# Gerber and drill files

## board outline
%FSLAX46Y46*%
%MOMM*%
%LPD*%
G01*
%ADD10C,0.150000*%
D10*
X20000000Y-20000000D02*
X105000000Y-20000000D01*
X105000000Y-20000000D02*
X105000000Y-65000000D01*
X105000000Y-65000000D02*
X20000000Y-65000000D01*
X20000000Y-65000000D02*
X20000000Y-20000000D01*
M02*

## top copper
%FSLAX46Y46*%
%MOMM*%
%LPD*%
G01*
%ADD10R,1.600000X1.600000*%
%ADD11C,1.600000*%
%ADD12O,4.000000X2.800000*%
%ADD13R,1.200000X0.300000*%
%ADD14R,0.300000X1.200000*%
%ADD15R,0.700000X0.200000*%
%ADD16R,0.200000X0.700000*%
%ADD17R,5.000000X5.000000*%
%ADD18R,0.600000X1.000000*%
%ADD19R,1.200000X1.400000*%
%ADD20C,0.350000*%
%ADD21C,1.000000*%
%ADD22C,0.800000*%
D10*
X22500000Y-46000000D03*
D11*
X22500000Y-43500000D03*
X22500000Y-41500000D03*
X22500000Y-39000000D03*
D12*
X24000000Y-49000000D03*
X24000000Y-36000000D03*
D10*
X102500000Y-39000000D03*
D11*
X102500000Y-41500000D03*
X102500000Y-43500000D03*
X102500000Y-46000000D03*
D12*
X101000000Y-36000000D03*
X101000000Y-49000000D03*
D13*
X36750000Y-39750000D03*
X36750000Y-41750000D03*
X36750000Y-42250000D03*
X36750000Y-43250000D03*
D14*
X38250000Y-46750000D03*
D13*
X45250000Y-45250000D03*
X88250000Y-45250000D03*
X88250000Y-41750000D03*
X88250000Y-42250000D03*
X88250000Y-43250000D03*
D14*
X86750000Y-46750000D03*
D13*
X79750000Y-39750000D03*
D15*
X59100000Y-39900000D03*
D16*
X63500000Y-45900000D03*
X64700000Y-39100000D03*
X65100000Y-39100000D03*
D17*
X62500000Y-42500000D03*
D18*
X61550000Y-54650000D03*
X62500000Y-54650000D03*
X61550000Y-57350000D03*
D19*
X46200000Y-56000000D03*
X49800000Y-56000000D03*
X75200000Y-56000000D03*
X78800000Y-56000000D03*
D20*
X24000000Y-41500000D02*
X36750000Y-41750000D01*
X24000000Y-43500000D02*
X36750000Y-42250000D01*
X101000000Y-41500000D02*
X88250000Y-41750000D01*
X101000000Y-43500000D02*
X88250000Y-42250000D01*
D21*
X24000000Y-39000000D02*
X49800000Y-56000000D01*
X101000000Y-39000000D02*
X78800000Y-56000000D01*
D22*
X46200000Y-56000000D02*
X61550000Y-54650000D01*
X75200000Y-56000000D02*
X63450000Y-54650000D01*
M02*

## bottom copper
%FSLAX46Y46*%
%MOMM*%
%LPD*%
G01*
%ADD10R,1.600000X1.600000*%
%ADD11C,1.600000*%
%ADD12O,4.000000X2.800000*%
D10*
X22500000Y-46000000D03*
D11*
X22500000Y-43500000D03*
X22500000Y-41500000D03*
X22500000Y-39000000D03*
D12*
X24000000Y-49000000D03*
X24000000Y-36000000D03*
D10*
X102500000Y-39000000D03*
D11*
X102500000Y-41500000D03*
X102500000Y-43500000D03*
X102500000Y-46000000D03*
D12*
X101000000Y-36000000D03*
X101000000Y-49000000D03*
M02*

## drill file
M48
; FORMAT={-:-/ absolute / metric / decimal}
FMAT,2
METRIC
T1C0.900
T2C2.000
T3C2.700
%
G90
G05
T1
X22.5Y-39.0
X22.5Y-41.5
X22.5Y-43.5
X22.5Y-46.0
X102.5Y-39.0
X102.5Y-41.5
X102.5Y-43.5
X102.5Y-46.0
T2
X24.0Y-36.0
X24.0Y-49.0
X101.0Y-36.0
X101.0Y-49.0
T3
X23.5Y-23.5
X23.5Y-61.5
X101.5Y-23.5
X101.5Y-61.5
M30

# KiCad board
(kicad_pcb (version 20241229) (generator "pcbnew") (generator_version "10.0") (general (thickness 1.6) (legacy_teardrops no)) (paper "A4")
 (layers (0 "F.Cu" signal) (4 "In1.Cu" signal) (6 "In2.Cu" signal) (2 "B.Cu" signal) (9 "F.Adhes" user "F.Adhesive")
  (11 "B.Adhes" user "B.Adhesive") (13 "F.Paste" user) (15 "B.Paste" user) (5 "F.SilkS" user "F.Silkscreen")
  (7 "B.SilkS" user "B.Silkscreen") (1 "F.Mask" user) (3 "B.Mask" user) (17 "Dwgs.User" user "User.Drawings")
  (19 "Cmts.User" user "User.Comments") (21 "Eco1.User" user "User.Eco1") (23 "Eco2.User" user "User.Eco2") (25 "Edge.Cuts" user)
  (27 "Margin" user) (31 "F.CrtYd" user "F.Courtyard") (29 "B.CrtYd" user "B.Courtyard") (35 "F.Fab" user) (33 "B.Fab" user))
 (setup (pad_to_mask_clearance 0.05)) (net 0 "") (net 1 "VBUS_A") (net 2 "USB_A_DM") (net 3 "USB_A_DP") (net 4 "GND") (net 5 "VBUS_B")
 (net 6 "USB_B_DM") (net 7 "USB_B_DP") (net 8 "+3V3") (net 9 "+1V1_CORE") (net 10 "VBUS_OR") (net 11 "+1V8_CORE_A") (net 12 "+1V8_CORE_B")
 (gr_line (start 20.0 20.0) (end 105.0 20.0) (layer "Edge.Cuts") (width 0.15))
 (gr_line (start 105.0 20.0) (end 105.0 65.0) (layer "Edge.Cuts") (width 0.15))
 (gr_line (start 105.0 65.0) (end 20.0 65.0) (layer "Edge.Cuts") (width 0.15))
 (gr_line (start 20.0 65.0) (end 20.0 20.0) (layer "Edge.Cuts") (width 0.15))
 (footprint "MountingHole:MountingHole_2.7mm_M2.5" (layer "F.Cu") (at 23.5 23.5)
  (pad "1" np_thru_hole circle (at 0 0) (size 2.7 2.7) (drill 2.7) (layers "*.Mask")))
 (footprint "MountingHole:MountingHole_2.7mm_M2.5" (layer "F.Cu") (at 101.5 23.5)
  (pad "1" np_thru_hole circle (at 0 0) (size 2.7 2.7) (drill 2.7) (layers "*.Mask")))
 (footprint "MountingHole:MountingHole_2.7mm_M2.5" (layer "F.Cu") (at 23.5 61.5)
  (pad "1" np_thru_hole circle (at 0 0) (size 2.7 2.7) (drill 2.7) (layers "*.Mask")))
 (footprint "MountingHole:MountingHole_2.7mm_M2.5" (layer "F.Cu") (at 101.5 61.5)
  (pad "1" np_thru_hole circle (at 0 0) (size 2.7 2.7) (drill 2.7) (layers "*.Mask")))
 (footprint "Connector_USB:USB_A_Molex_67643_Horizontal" (layer "F.Cu") (at 24.0 42.5 90)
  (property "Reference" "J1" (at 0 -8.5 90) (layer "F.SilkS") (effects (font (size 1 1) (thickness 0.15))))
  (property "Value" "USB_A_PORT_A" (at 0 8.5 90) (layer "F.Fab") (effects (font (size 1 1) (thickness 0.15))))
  (pad "1" thru_hole rect (at -3.5 -1.5 90) (size 1.6 1.6) (drill 0.9) (layers "*.Cu" "*.Mask") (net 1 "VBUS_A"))
  (pad "2" thru_hole circle (at -1.0 -1.5 90) (size 1.6 1.6) (drill 0.9) (layers "*.Cu" "*.Mask") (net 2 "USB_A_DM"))
  (pad "3" thru_hole circle (at 1.0 -1.5 90) (size 1.6 1.6) (drill 0.9) (layers "*.Cu" "*.Mask") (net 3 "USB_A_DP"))
  (pad "4" thru_hole circle (at 3.5 -1.5 90) (size 1.6 1.6) (drill 0.9) (layers "*.Cu" "*.Mask") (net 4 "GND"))
  (pad "SH1" thru_hole oval (at -6.5 0 90) (size 2.8 4.0) (drill 2.0 3.2) (layers "*.Cu" "*.Mask") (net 4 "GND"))
  (pad "SH2" thru_hole oval (at 6.5 0 90) (size 2.8 4.0) (drill 2.0 3.2) (layers "*.Cu" "*.Mask") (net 4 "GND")))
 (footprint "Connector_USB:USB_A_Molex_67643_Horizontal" (layer "F.Cu") (at 101.0 42.5 270)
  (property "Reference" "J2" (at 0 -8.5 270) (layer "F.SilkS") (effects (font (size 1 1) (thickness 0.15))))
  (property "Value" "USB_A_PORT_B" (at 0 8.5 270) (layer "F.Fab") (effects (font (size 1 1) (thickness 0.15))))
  (pad "1" thru_hole rect (at -3.5 -1.5 270) (size 1.6 1.6) (drill 0.9) (layers "*.Cu" "*.Mask") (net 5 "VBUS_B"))
  (pad "2" thru_hole circle (at -1.0 -1.5 270) (size 1.6 1.6) (drill 0.9) (layers "*.Cu" "*.Mask") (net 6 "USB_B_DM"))
  (pad "3" thru_hole circle (at 1.0 -1.5 270) (size 1.6 1.6) (drill 0.9) (layers "*.Cu" "*.Mask") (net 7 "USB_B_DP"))
  (pad "4" thru_hole circle (at 3.5 -1.5 270) (size 1.6 1.6) (drill 0.9) (layers "*.Cu" "*.Mask") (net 4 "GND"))
  (pad "SH1" thru_hole oval (at -6.5 0 270) (size 2.8 4.0) (drill 2.0 3.2) (layers "*.Cu" "*.Mask") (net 4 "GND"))
  (pad "SH2" thru_hole oval (at 6.5 0 270) (size 2.8 4.0) (drill 2.0 3.2) (layers "*.Cu" "*.Mask") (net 4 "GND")))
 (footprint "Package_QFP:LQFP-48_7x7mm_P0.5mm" (layer "F.Cu") (at 41.0 42.5)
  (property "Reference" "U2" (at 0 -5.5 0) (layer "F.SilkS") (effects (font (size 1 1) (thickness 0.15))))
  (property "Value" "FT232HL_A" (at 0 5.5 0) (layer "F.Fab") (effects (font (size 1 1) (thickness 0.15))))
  (pad "1" smd rect (at -4.25 -2.75) (size 1.2 0.3) (layers "F.Cu" "F.Paste" "F.Mask") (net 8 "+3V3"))
  (pad "7" smd rect (at -4.25 -0.75) (size 1.2 0.3) (layers "F.Cu" "F.Paste" "F.Mask") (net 2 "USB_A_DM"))
  (pad "8" smd rect (at -4.25 -0.25) (size 1.2 0.3) (layers "F.Cu" "F.Paste" "F.Mask") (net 3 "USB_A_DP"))
  (pad "10" smd rect (at -4.25 0.75) (size 1.2 0.3) (layers "F.Cu" "F.Paste" "F.Mask") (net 4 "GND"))
  (pad "13" smd rect (at -2.75 4.25 90) (size 1.2 0.3) (layers "F.Cu" "F.Paste" "F.Mask") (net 8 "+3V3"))
  (pad "25" smd rect (at 4.25 2.75) (size 1.2 0.3) (layers "F.Cu" "F.Paste" "F.Mask") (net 4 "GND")))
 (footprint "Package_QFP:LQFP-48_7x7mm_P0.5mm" (layer "F.Cu") (at 84.0 42.5)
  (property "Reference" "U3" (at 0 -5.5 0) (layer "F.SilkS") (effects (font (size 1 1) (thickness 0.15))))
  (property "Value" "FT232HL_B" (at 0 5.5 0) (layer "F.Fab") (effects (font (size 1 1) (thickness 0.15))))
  (pad "1" smd rect (at 4.25 2.75) (size 1.2 0.3) (layers "F.Cu" "F.Paste" "F.Mask") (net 8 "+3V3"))
  (pad "7" smd rect (at 4.25 -0.75) (size 1.2 0.3) (layers "F.Cu" "F.Paste" "F.Mask") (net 6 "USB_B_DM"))
  (pad "8" smd rect (at 4.25 -0.25) (size 1.2 0.3) (layers "F.Cu" "F.Paste" "F.Mask") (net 7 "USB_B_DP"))
  (pad "10" smd rect (at 4.25 0.75) (size 1.2 0.3) (layers "F.Cu" "F.Paste" "F.Mask") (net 4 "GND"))
  (pad "13" smd rect (at 2.75 4.25 90) (size 1.2 0.3) (layers "F.Cu" "F.Paste" "F.Mask") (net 8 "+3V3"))
  (pad "25" smd rect (at -4.25 -2.75) (size 1.2 0.3) (layers "F.Cu" "F.Paste" "F.Mask") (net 4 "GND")))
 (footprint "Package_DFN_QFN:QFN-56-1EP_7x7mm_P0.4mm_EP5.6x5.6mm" (layer "F.Cu") (at 62.5 42.5)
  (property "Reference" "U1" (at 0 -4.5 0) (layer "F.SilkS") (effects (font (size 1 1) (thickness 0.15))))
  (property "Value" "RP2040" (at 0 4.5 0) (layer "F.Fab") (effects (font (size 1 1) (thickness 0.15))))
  (pad "1" smd rect (at -3.4 -2.6) (size 0.7 0.2) (layers "F.Cu" "F.Paste" "F.Mask") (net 8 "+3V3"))
  (pad "19" smd rect (at 1.0 3.4 90) (size 0.7 0.2) (layers "F.Cu" "F.Paste" "F.Mask") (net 4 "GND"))
  (pad "44" smd rect (at 2.2 -3.4 90) (size 0.7 0.2) (layers "F.Cu" "F.Paste" "F.Mask") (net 8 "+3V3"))
  (pad "45" smd rect (at 2.6 -3.4 90) (size 0.7 0.2) (layers "F.Cu" "F.Paste" "F.Mask") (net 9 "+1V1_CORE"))
  (pad "57" smd rect (at 0 0) (size 5.0 5.0) (layers "F.Cu" "F.Paste" "F.Mask") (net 4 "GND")))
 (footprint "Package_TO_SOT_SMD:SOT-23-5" (layer "F.Cu") (at 62.5 56.0)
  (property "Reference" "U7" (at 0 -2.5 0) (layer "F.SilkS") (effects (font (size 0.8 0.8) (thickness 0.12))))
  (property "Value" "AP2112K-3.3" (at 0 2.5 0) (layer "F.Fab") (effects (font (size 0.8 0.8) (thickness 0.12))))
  (pad "1" smd rect (at -0.95 -1.35) (size 0.6 1.0) (layers "F.Cu" "F.Paste" "F.Mask") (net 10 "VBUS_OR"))
  (pad "2" smd rect (at 0 -1.35) (size 0.6 1.0) (layers "F.Cu" "F.Paste" "F.Mask") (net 4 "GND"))
  (pad "5" smd rect (at -0.95 1.35) (size 0.6 1.0) (layers "F.Cu" "F.Paste" "F.Mask") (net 8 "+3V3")))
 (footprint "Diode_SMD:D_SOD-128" (layer "F.Cu") (at 48.0 56.0)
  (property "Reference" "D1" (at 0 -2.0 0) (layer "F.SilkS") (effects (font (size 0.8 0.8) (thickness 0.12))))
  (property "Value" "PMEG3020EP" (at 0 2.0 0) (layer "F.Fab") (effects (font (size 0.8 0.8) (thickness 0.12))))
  (pad "1" smd rect (at -1.8 0) (size 1.2 1.4) (layers "F.Cu" "F.Paste" "F.Mask") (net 10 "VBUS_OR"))
  (pad "2" smd rect (at 1.8 0) (size 1.2 1.4) (layers "F.Cu" "F.Paste" "F.Mask") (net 1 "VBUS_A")))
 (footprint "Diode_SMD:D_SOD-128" (layer "F.Cu") (at 77.0 56.0)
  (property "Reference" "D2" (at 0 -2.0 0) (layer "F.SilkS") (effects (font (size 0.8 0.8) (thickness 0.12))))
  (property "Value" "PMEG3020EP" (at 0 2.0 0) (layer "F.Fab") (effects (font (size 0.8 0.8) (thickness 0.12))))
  (pad "1" smd rect (at -1.8 0) (size 1.2 1.4) (layers "F.Cu" "F.Paste" "F.Mask") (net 10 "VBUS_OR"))
  (pad "2" smd rect (at 1.8 0) (size 1.2 1.4) (layers "F.Cu" "F.Paste" "F.Mask") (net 5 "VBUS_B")))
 (segment (start 24.0 41.5) (end 36.75 41.75) (width 0.35) (layer "F.Cu") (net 2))
 (segment (start 24.0 43.5) (end 36.75 42.25) (width 0.35) (layer "F.Cu") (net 3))
 (segment (start 101.0 41.5) (end 88.25 41.75) (width 0.35) (layer "F.Cu") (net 6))
 (segment (start 101.0 43.5) (end 88.25 42.25) (width 0.35) (layer "F.Cu") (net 7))
 (segment (start 24.0 39.0) (end 49.8 56.0) (width 1.0) (layer "F.Cu") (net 1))
 (segment (start 101.0 39.0) (end 78.8 56.0) (width 1.0) (layer "F.Cu") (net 5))
 (segment (start 46.2 56.0) (end 61.55 54.65) (width 0.8) (layer "F.Cu") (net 10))
 (segment (start 75.2 56.0) (end 63.45 54.65) (width 0.8) (layer "F.Cu") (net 10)))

